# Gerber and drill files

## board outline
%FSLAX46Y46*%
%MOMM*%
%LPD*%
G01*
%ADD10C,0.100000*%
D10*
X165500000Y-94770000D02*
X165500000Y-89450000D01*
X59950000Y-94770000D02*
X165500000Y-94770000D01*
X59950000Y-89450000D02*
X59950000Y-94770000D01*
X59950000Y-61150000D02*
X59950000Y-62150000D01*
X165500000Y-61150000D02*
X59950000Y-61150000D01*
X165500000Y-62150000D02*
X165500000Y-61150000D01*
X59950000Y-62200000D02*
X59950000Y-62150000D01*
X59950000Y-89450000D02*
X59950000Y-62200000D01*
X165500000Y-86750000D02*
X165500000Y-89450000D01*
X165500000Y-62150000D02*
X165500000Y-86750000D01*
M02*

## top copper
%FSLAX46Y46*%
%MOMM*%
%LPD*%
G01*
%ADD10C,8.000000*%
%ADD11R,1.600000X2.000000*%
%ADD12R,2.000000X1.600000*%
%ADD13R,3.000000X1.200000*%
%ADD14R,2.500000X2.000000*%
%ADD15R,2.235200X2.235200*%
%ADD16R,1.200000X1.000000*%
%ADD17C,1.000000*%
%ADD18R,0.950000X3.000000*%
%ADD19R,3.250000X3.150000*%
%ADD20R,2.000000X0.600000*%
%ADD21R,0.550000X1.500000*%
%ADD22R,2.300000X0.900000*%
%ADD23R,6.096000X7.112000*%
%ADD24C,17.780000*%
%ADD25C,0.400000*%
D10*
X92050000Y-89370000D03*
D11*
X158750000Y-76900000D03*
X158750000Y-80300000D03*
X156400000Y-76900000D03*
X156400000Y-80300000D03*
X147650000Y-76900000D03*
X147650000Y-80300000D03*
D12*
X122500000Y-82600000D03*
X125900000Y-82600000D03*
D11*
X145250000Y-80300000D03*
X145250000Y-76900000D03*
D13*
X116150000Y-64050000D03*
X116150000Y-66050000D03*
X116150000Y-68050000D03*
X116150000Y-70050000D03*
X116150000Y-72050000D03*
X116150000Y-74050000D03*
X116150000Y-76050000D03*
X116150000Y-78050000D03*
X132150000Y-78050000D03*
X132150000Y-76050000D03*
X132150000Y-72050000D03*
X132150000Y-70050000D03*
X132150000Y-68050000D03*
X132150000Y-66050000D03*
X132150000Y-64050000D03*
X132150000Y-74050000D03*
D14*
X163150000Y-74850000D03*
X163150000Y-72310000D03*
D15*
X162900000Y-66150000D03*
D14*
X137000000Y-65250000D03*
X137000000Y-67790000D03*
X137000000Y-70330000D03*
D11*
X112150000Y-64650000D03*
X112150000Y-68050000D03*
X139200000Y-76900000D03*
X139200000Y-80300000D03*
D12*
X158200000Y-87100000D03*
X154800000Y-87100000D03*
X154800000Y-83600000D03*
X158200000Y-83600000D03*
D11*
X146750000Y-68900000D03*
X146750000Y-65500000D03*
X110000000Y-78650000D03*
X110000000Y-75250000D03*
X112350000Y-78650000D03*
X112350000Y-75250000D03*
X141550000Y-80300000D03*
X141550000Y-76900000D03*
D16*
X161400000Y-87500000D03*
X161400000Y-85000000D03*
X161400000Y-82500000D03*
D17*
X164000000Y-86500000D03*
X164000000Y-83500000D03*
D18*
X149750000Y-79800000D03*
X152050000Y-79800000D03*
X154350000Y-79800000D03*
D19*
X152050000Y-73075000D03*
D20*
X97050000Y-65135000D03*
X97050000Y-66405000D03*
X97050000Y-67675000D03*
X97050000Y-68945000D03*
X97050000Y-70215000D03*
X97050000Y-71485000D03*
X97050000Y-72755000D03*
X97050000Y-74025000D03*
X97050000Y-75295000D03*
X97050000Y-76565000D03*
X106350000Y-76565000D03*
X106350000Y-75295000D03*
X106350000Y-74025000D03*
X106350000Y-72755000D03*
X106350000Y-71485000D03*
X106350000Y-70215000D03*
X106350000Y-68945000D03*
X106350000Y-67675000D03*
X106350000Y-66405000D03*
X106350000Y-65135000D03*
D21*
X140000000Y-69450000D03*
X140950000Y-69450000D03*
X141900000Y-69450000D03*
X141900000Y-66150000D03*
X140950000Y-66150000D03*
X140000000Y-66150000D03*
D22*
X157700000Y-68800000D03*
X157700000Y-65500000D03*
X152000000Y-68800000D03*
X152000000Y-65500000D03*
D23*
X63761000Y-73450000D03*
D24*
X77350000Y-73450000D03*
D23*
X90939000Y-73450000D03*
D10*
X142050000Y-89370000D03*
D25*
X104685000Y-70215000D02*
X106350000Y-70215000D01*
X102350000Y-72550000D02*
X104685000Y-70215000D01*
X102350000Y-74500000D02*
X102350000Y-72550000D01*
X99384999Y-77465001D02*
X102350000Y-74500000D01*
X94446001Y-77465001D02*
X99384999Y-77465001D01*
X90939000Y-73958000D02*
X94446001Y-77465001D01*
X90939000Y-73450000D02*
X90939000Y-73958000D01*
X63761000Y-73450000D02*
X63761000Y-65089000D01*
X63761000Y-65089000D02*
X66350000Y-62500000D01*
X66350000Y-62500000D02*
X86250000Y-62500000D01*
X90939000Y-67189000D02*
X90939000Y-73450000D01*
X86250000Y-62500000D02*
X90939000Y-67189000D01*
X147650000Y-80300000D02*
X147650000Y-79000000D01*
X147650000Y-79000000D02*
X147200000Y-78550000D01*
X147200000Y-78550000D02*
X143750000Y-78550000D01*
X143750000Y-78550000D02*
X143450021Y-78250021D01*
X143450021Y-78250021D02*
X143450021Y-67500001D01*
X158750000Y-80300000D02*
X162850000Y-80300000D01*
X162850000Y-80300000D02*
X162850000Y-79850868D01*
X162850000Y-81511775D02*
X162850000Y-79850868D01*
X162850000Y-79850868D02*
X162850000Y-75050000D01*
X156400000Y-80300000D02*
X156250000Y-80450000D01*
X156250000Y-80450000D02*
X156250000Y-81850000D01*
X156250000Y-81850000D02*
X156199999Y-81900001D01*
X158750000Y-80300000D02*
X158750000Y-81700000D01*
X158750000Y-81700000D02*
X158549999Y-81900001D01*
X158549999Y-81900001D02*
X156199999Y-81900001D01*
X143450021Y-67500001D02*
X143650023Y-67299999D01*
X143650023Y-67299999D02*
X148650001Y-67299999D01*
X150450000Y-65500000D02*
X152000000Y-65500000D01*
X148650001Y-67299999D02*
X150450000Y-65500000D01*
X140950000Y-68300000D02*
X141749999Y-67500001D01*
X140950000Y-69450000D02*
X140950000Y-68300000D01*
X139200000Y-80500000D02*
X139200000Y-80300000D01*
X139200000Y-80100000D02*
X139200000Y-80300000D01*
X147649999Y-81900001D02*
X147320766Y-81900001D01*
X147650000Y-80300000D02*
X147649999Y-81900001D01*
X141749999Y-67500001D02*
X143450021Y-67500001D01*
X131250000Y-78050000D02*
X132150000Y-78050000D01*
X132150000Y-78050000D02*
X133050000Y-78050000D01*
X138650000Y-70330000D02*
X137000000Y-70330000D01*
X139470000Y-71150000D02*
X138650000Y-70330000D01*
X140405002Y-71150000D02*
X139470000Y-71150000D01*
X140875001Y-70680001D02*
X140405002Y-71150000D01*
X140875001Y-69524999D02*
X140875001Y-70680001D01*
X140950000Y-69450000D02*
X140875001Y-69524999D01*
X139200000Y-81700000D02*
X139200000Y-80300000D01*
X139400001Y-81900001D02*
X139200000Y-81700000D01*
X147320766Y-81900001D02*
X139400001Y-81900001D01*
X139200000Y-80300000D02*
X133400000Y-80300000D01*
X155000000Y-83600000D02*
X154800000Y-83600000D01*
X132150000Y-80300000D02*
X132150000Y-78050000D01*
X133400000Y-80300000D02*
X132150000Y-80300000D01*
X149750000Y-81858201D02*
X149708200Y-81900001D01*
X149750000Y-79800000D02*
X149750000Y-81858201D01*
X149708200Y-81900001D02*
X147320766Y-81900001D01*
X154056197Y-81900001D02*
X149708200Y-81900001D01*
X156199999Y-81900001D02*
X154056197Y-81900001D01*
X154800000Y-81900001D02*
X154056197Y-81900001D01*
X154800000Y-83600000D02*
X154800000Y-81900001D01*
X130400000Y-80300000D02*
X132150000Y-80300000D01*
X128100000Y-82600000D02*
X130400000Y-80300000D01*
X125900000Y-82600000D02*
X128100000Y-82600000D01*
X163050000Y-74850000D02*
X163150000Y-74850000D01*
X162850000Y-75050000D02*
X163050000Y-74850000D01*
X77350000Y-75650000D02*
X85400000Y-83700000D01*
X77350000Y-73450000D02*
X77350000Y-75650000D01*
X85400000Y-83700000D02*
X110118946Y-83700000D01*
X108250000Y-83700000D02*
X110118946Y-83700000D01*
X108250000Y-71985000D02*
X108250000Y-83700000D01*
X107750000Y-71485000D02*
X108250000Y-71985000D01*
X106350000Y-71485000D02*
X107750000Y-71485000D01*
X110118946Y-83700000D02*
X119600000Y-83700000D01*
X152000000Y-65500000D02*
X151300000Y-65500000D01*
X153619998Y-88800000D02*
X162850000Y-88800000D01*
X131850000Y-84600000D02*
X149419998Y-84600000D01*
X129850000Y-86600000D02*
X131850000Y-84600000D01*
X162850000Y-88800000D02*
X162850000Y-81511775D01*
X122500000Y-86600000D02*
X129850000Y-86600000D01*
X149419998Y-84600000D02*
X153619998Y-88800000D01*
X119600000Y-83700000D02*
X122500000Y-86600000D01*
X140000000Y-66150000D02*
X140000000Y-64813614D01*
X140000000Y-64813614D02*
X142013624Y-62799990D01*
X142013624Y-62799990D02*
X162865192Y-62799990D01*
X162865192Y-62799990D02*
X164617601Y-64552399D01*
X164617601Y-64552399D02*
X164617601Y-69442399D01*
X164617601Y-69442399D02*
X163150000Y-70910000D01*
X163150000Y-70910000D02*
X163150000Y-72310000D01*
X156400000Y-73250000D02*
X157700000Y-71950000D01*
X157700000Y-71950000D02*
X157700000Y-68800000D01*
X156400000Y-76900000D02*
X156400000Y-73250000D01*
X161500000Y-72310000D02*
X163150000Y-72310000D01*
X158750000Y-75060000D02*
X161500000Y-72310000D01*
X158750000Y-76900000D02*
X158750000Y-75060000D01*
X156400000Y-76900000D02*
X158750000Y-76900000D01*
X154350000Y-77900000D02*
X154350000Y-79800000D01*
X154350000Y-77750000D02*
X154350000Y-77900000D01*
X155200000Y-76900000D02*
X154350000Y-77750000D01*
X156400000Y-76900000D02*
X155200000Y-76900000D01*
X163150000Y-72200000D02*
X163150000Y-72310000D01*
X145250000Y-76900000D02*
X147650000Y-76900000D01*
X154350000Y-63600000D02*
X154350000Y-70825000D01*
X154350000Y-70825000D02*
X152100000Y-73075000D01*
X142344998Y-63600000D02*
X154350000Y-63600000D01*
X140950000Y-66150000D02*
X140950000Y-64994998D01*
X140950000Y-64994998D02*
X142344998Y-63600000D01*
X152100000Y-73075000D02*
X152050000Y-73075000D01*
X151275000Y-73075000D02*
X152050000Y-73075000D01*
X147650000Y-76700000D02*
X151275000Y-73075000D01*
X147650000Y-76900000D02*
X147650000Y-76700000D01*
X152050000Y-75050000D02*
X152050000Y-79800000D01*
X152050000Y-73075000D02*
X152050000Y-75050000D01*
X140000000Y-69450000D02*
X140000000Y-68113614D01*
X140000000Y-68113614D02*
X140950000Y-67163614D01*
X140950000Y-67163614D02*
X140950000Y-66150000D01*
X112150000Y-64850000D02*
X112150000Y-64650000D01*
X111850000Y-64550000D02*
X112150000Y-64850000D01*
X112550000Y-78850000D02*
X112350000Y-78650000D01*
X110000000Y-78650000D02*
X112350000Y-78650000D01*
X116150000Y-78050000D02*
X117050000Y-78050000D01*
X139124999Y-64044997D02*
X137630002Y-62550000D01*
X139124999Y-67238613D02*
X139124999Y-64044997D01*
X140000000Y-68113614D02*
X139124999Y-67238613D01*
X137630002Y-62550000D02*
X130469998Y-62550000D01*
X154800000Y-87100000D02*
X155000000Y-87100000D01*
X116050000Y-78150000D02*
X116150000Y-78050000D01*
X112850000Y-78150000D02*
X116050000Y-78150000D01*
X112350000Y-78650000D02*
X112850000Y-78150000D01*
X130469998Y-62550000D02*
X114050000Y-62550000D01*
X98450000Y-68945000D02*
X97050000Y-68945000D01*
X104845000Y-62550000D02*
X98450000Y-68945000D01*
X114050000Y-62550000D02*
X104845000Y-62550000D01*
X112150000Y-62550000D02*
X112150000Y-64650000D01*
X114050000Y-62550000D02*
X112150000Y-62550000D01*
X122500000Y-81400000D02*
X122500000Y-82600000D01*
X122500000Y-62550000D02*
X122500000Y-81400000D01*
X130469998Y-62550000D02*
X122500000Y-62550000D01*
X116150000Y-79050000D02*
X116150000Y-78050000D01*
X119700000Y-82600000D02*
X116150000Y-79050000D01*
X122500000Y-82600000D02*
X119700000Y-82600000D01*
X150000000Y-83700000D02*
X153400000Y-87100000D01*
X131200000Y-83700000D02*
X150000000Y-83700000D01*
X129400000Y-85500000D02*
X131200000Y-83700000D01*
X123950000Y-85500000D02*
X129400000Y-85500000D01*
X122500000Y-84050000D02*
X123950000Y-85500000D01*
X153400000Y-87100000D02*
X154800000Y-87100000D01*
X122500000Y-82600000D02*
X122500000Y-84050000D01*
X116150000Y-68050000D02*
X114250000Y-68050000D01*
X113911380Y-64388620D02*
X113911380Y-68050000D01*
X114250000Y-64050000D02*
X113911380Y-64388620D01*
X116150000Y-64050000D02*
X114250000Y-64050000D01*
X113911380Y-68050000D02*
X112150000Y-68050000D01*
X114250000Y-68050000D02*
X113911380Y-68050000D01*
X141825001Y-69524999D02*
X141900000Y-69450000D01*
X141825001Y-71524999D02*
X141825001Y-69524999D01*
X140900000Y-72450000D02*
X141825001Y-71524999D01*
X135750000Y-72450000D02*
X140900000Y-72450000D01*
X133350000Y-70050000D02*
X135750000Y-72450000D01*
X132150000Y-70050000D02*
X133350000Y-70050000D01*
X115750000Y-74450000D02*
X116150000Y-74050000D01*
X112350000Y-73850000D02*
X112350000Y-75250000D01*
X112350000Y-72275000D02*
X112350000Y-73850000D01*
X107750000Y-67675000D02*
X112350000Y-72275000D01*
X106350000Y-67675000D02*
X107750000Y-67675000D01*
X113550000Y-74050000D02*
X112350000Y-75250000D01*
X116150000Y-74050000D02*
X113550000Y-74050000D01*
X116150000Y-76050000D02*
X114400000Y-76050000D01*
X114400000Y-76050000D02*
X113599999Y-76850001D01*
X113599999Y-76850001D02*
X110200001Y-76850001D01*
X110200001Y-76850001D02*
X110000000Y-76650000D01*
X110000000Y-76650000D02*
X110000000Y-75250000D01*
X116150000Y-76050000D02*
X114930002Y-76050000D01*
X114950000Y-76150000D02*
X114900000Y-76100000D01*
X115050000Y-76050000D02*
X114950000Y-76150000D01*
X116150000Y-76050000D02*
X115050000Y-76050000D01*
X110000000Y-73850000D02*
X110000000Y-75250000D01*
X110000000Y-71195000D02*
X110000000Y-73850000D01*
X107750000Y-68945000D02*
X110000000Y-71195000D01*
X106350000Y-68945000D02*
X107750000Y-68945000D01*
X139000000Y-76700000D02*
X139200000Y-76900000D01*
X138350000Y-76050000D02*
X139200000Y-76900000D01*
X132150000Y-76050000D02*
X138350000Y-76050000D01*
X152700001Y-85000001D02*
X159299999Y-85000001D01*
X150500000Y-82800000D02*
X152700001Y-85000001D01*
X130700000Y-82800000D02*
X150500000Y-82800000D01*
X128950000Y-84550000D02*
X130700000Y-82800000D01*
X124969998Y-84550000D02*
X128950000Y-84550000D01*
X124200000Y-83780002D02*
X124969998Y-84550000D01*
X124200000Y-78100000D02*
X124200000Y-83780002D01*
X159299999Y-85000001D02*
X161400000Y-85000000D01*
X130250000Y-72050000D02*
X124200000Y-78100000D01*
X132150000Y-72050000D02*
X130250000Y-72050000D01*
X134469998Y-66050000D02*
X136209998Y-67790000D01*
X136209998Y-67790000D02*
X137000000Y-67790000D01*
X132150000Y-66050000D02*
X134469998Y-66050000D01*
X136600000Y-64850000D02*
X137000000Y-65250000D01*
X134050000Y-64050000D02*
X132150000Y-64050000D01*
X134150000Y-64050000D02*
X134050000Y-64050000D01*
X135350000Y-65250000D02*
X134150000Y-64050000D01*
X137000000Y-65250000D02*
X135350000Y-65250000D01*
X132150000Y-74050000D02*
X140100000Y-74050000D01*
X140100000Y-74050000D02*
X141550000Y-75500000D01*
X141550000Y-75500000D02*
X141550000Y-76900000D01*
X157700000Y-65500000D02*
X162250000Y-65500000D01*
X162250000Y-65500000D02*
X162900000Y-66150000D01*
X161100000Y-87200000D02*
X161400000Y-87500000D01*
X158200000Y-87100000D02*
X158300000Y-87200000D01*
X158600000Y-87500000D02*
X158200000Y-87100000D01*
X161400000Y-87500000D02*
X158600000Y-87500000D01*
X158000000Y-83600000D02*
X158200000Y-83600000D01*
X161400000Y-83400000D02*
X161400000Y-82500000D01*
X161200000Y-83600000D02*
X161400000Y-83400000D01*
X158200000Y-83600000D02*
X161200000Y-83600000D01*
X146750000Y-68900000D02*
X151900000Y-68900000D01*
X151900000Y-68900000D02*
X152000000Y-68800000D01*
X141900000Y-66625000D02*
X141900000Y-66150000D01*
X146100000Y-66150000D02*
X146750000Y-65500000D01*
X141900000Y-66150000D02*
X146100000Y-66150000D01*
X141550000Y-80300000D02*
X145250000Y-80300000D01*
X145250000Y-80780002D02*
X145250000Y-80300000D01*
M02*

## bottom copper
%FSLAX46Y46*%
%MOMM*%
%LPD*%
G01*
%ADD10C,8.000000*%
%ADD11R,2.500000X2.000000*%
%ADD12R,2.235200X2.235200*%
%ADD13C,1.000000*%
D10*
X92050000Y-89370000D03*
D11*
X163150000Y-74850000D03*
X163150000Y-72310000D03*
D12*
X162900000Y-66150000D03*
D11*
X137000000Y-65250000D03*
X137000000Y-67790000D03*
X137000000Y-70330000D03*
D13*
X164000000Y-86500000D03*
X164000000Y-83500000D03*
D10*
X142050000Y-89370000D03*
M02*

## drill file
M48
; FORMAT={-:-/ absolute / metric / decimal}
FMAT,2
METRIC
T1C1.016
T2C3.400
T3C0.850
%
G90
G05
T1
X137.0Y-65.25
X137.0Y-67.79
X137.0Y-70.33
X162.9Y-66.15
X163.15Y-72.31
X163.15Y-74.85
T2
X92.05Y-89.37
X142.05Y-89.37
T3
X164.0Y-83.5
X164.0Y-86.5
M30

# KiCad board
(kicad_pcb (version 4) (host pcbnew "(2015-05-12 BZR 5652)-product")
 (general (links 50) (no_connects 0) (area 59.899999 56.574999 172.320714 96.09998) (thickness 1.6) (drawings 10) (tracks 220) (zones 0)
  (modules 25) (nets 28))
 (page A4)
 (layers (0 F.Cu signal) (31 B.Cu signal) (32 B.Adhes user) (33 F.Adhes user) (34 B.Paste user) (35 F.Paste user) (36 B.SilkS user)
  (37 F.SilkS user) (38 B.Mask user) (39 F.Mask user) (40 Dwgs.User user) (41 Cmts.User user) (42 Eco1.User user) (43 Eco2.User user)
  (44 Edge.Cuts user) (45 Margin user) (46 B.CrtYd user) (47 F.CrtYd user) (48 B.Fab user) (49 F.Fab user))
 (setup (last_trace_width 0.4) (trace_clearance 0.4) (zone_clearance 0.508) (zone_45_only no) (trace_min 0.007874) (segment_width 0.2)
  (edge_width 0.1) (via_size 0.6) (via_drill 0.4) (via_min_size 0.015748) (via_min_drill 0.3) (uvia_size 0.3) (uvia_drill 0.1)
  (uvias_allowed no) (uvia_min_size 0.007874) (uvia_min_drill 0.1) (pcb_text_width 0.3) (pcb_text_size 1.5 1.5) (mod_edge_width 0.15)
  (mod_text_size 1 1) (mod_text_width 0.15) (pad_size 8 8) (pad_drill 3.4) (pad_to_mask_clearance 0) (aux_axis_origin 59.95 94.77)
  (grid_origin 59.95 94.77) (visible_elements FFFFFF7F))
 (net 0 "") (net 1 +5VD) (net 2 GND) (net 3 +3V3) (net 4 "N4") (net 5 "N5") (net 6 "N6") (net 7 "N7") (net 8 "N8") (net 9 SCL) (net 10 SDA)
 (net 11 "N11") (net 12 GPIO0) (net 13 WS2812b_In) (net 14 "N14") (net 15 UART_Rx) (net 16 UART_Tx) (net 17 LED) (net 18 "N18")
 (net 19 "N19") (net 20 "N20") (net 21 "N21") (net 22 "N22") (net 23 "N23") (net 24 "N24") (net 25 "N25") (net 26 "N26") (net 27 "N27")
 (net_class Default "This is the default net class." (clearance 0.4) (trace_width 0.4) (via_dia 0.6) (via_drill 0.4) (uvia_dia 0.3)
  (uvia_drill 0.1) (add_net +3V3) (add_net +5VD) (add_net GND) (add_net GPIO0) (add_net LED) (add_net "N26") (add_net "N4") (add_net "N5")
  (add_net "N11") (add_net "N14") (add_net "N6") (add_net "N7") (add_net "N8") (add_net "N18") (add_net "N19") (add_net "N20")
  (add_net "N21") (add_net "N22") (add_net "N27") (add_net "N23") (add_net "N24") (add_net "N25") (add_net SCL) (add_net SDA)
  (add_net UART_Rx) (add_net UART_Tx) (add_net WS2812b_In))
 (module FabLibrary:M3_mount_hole (layer F.Cu) (at 92.05 89.37)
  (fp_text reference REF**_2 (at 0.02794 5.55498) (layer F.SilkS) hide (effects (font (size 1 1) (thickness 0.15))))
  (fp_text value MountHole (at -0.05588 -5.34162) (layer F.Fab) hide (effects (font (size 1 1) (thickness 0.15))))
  (pad 1 thru_hole circle (at 0 0) (size 8 8) (drill 3.4) (layers *.Cu *.Mask F.SilkS)))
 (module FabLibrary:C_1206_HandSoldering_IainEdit (layer F.Cu) (at 158.75 78.6 270)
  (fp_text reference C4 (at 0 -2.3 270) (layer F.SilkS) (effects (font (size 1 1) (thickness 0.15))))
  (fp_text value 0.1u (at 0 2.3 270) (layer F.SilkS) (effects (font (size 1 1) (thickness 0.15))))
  (pad 1 smd rect (at -1.7 0 270) (size 2 1.6) (layers F.Cu F.Paste F.Mask) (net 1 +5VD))
  (pad 2 smd rect (at 1.7 0 270) (size 2 1.6) (layers F.Cu F.Paste F.Mask) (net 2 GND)))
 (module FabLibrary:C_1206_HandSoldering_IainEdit (layer F.Cu) (at 156.4 78.6 270)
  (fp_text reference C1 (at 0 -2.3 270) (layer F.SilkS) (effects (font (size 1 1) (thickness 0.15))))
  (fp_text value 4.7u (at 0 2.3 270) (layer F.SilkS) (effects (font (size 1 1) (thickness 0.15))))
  (pad 1 smd rect (at -1.7 0 270) (size 2 1.6) (layers F.Cu F.Paste F.Mask) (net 1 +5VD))
  (pad 2 smd rect (at 1.7 0 270) (size 2 1.6) (layers F.Cu F.Paste F.Mask) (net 2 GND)))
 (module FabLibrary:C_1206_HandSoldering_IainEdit (layer F.Cu) (at 147.65 78.6 270)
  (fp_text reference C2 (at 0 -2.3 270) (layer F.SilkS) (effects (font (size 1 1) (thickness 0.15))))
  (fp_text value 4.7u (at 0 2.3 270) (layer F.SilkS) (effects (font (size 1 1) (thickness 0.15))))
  (pad 1 smd rect (at -1.7 0 270) (size 2 1.6) (layers F.Cu F.Paste F.Mask) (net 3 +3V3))
  (pad 2 smd rect (at 1.7 0 270) (size 2 1.6) (layers F.Cu F.Paste F.Mask) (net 2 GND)))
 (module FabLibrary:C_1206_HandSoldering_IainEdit (layer F.Cu) (at 124.2 82.6)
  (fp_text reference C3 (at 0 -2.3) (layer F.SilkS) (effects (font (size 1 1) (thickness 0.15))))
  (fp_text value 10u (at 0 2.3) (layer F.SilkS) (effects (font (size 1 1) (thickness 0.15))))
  (pad 1 smd rect (at -1.7 0) (size 2 1.6) (layers F.Cu F.Paste F.Mask) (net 3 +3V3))
  (pad 2 smd rect (at 1.7 0) (size 2 1.6) (layers F.Cu F.Paste F.Mask) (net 2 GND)))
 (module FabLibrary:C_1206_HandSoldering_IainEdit (layer F.Cu) (at 145.25 78.6 90)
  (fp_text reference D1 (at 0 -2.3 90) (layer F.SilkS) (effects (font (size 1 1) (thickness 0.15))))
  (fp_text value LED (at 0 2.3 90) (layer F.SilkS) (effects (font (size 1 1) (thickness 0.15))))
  (pad 1 smd rect (at -1.7 0 90) (size 2 1.6) (layers F.Cu F.Paste F.Mask) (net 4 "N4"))
  (pad 2 smd rect (at 1.7 0 90) (size 2 1.6) (layers F.Cu F.Paste F.Mask) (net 3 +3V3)))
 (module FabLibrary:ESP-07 (layer F.Cu) (at 124.15 70.05 270)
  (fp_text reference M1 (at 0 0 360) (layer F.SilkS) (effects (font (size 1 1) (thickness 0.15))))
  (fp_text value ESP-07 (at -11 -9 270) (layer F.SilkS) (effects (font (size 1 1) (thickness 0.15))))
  (pad 1 smd rect (at -6 8 270) (size 1.2 3) (layers F.Cu F.Paste F.Mask) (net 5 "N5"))
  (pad 2 smd rect (at -4 8 270) (size 1.2 3) (layers F.Cu F.Paste F.Mask) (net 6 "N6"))
  (pad 3 smd rect (at -2 8 270) (size 1.2 3) (layers F.Cu F.Paste F.Mask) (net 5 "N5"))
  (pad 4 smd rect (at 0 8 270) (size 1.2 3) (layers F.Cu F.Paste F.Mask) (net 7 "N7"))
  (pad 5 smd rect (at 2 8 270) (size 1.2 3) (layers F.Cu F.Paste F.Mask) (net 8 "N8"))
  (pad 6 smd rect (at 4 8 270) (size 1.2 3) (layers F.Cu F.Paste F.Mask) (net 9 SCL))
  (pad 7 smd rect (at 6 8 270) (size 1.2 3) (layers F.Cu F.Paste F.Mask) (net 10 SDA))
  (pad 8 smd rect (at 8 8 270) (size 1.2 3) (layers F.Cu F.Paste F.Mask) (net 3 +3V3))
  (pad 9 smd rect (at 8 -8 270) (size 1.2 3) (layers F.Cu F.Paste F.Mask) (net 2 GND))
  (pad 10 smd rect (at 6 -8 270) (size 1.2 3) (layers F.Cu F.Paste F.Mask) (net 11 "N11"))
  (pad 12 smd rect (at 2 -8 270) (size 1.2 3) (layers F.Cu F.Paste F.Mask) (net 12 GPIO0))
  (pad 13 smd rect (at 0 -8 270) (size 1.2 3) (layers F.Cu F.Paste F.Mask) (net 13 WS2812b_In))
  (pad 14 smd rect (at -2 -8 270) (size 1.2 3) (layers F.Cu F.Paste F.Mask) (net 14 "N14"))
  (pad 15 smd rect (at -4 -8 270) (size 1.2 3) (layers F.Cu F.Paste F.Mask) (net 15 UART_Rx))
  (pad 16 smd rect (at -6 -8 270) (size 1.2 3) (layers F.Cu F.Paste F.Mask) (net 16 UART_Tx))
  (pad 11 smd rect (at 4 -8 270) (size 1.2 3) (layers F.Cu F.Paste F.Mask) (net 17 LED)))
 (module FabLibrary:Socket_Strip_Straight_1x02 (layer F.Cu) (at 163.15 74.85 90)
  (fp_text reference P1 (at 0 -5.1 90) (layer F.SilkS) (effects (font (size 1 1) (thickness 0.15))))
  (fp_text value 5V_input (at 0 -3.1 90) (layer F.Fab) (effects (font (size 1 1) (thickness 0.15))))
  (pad 1 thru_hole rect (at 0 0 90) (size 2 2.5) (drill 1.016) (layers *.Mask F.Cu F.SilkS) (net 2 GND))
  (pad 2 thru_hole rect (at 2.54 0 90) (size 2 2.5) (drill 1.016) (layers *.Mask F.Cu F.SilkS) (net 1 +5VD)))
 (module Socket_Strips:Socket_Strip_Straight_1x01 (layer F.Cu) (at 162.9 66.15)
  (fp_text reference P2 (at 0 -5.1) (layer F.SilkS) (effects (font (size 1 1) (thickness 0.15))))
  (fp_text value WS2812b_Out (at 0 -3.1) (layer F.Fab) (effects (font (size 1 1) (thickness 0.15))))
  (pad 1 thru_hole rect (at 0 0) (size 2.2352 2.2352) (drill 1.016) (layers *.Cu *.Mask F.SilkS) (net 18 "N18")))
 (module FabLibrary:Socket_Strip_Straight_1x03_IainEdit (layer F.Cu) (at 137 65.25 270)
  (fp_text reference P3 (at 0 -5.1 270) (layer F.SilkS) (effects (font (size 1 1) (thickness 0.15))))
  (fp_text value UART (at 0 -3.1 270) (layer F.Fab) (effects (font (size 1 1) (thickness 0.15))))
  (pad 1 thru_hole rect (at 0 0 270) (size 2 2.5) (drill 1.016) (layers *.Mask F.Cu F.SilkS) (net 16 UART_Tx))
  (pad 2 thru_hole rect (at 2.54 0 270) (size 2 2.5) (drill 1.016) (layers *.Mask F.Cu F.SilkS) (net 15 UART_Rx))
  (pad 3 thru_hole rect (at 5.08 0 270) (size 2 2.5) (drill 1.016) (layers *.Mask F.Cu F.SilkS) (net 2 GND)))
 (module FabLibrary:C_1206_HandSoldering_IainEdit (layer F.Cu) (at 112.15 66.35 270)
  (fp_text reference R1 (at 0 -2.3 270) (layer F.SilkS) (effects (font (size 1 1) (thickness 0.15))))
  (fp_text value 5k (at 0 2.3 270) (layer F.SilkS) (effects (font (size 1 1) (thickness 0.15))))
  (pad 1 smd rect (at -1.7 0 270) (size 2 1.6) (layers F.Cu F.Paste F.Mask) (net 3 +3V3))
  (pad 2 smd rect (at 1.7 0 270) (size 2 1.6) (layers F.Cu F.Paste F.Mask) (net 5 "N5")))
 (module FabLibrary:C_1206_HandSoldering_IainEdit (layer F.Cu) (at 139.2 78.6 270)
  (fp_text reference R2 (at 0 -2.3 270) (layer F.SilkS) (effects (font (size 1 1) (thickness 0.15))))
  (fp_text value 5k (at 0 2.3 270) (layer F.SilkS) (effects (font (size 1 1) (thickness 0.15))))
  (pad 1 smd rect (at -1.7 0 270) (size 2 1.6) (layers F.Cu F.Paste F.Mask) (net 11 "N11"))
  (pad 2 smd rect (at 1.7 0 270) (size 2 1.6) (layers F.Cu F.Paste F.Mask) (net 2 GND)))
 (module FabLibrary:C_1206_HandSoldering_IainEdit (layer F.Cu) (at 156.5 87.1 180)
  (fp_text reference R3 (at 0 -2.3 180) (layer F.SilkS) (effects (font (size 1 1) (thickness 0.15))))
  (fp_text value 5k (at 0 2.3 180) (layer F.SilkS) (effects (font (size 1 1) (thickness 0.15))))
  (pad 1 smd rect (at -1.7 0 180) (size 2 1.6) (layers F.Cu F.Paste F.Mask) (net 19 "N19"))
  (pad 2 smd rect (at 1.7 0 180) (size 2 1.6) (layers F.Cu F.Paste F.Mask) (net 3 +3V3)))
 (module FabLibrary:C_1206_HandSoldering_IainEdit (layer F.Cu) (at 156.5 83.6)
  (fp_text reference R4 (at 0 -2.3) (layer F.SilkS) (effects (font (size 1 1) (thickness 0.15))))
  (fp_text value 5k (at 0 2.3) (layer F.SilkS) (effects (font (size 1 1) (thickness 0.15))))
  (pad 1 smd rect (at -1.7 0) (size 2 1.6) (layers F.Cu F.Paste F.Mask) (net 2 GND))
  (pad 2 smd rect (at 1.7 0) (size 2 1.6) (layers F.Cu F.Paste F.Mask) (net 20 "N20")))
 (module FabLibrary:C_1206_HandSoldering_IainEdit (layer F.Cu) (at 146.75 67.2 90)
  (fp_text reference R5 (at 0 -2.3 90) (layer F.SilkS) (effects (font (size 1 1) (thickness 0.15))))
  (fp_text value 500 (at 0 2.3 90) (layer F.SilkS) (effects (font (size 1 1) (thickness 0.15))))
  (pad 1 smd rect (at -1.7 0 90) (size 2 1.6) (layers F.Cu F.Paste F.Mask) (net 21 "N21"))
  (pad 2 smd rect (at 1.7 0 90) (size 2 1.6) (layers F.Cu F.Paste F.Mask) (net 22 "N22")))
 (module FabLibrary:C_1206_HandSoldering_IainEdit (layer F.Cu) (at 110 76.95 90)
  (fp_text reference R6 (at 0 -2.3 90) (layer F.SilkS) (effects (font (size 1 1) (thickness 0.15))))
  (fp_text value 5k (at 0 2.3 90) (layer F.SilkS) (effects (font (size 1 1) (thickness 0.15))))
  (pad 1 smd rect (at -1.7 0 90) (size 2 1.6) (layers F.Cu F.Paste F.Mask) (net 3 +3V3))
  (pad 2 smd rect (at 1.7 0 90) (size 2 1.6) (layers F.Cu F.Paste F.Mask) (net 10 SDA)))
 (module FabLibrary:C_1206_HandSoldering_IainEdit (layer F.Cu) (at 112.35 76.95 90)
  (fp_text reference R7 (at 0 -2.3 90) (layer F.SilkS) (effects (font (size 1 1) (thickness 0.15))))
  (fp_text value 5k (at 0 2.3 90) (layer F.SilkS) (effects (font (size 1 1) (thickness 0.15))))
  (pad 1 smd rect (at -1.7 0 90) (size 2 1.6) (layers F.Cu F.Paste F.Mask) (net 3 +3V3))
  (pad 2 smd rect (at 1.7 0 90) (size 2 1.6) (layers F.Cu F.Paste F.Mask) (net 9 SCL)))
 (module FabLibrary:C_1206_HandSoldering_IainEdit (layer F.Cu) (at 141.55 78.6 90)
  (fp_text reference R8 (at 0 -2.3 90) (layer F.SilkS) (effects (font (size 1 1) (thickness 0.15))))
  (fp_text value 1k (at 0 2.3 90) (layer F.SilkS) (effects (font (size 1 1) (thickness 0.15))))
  (pad 1 smd rect (at -1.7 0 90) (size 2 1.6) (layers F.Cu F.Paste F.Mask) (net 4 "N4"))
  (pad 2 smd rect (at 1.7 0 90) (size 2 1.6) (layers F.Cu F.Paste F.Mask) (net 17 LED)))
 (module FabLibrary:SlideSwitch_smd (layer F.Cu) (at 164 85 90)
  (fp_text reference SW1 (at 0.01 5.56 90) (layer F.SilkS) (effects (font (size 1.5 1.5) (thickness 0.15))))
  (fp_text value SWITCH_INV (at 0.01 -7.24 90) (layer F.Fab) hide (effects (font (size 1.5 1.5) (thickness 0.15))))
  (pad 1 smd rect (at -2.5 -2.6 90) (size 1 1.2) (layers F.Cu F.Paste F.Mask) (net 19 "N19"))
  (pad 2 smd rect (at 0 -2.6 90) (size 1 1.2) (layers F.Cu F.Paste F.Mask) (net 12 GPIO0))
  (pad 3 smd rect (at 2.5 -2.6 90) (size 1 1.2) (layers F.Cu F.Paste F.Mask) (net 20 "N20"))
  (pad "" np_thru_hole circle (at -1.5 0 90) (size 1 1) (drill 0.85) (layers *.Cu *.Mask F.SilkS))
  (pad "" np_thru_hole circle (at 1.5 0 90) (size 1 1) (drill 0.85) (layers *.Cu *.Mask F.SilkS)))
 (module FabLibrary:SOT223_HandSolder (layer F.Cu) (at 152.05 78.3)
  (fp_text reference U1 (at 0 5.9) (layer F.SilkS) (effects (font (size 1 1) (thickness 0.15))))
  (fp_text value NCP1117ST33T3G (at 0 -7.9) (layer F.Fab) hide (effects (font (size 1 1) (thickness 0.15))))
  (pad 1 smd rect (at -2.3 1.5) (size 0.95 3) (layers F.Cu F.Paste F.Mask) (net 2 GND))
  (pad 2 smd rect (at 0 1.5) (size 0.95 3) (layers F.Cu F.Paste F.Mask) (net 3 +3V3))
  (pad 3 smd rect (at 2.3 1.5) (size 0.95 3) (layers F.Cu F.Paste F.Mask) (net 1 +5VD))
  (pad 2 smd rect (at 0 -5.225) (size 3.25 3.15) (layers F.Cu F.Paste F.Mask) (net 3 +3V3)))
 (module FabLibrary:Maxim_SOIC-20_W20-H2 (layer F.Cu) (at 101.7 70.85 270)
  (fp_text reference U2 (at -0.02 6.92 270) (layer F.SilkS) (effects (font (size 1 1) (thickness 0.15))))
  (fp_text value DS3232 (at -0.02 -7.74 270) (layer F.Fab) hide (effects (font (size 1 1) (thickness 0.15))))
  (pad 1 smd rect (at -5.715 4.65 270) (size 0.6 2) (layers F.Cu F.Paste F.Mask))
  (pad 2 smd rect (at -4.445 4.65 270) (size 0.6 2) (layers F.Cu F.Paste F.Mask))
  (pad 3 smd rect (at -3.175 4.65 270) (size 0.6 2) (layers F.Cu F.Paste F.Mask) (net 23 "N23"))
  (pad 4 smd rect (at -1.905 4.65 270) (size 0.6 2) (layers F.Cu F.Paste F.Mask) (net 3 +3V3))
  (pad 5 smd rect (at -0.635 4.65 270) (size 0.6 2) (layers F.Cu F.Paste F.Mask) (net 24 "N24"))
  (pad 6 smd rect (at 0.635 4.65 270) (size 0.6 2) (layers F.Cu F.Paste F.Mask) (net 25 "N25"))
  (pad 7 smd rect (at 1.905 4.65 270) (size 0.6 2) (layers F.Cu F.Paste F.Mask))
  (pad 8 smd rect (at 3.175 4.65 270) (size 0.6 2) (layers F.Cu F.Paste F.Mask))
  (pad 9 smd rect (at 4.445 4.65 270) (size 0.6 2) (layers F.Cu F.Paste F.Mask))
  (pad 10 smd rect (at 5.715 4.65 270) (size 0.6 2) (layers F.Cu F.Paste F.Mask))
  (pad 11 smd rect (at 5.715 -4.65 270) (size 0.6 2) (layers F.Cu F.Paste F.Mask))
  (pad 12 smd rect (at 4.445 -4.65 270) (size 0.6 2) (layers F.Cu F.Paste F.Mask))
  (pad 13 smd rect (at 3.175 -4.65 270) (size 0.6 2) (layers F.Cu F.Paste F.Mask))
  (pad 14 smd rect (at 1.905 -4.65 270) (size 0.6 2) (layers F.Cu F.Paste F.Mask))
  (pad 15 smd rect (at 0.635 -4.65 270) (size 0.6 2) (layers F.Cu F.Paste F.Mask) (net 2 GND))
  (pad 16 smd rect (at -0.635 -4.65 270) (size 0.6 2) (layers F.Cu F.Paste F.Mask) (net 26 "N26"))
  (pad 17 smd rect (at -1.905 -4.65 270) (size 0.6 2) (layers F.Cu F.Paste F.Mask) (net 10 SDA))
  (pad 18 smd rect (at -3.175 -4.65 270) (size 0.6 2) (layers F.Cu F.Paste F.Mask) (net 9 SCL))
  (pad 19 smd rect (at -4.445 -4.65 270) (size 0.6 2) (layers F.Cu F.Paste F.Mask))
  (pad 20 smd rect (at -5.715 -4.65 270) (size 0.6 2) (layers F.Cu F.Paste F.Mask) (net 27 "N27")))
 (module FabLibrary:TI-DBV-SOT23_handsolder (layer F.Cu) (at 140.95 67.85)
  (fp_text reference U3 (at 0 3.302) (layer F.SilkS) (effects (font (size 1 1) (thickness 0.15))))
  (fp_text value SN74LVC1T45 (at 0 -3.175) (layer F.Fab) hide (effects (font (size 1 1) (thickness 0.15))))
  (pad 1 smd rect (at -0.95 1.6) (size 0.55 1.5) (layers F.Cu F.Paste F.Mask) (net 3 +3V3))
  (pad 2 smd rect (at 0 1.6) (size 0.55 1.5) (layers F.Cu F.Paste F.Mask) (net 2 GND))
  (pad 3 smd rect (at 0.95 1.6) (size 0.55 1.5) (layers F.Cu F.Paste F.Mask) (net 13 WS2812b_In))
  (pad 4 smd rect (at 0.95 -1.7) (size 0.55 1.5) (layers F.Cu F.Paste F.Mask) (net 22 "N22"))
  (pad 5 smd rect (at 0 -1.7) (size 0.55 1.5) (layers F.Cu F.Paste F.Mask) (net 3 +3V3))
  (pad 6 smd rect (at -0.95 -1.7) (size 0.55 1.5) (layers F.Cu F.Paste F.Mask) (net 1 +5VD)))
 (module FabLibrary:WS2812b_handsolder (layer F.Cu) (at 154.85 67.15 180)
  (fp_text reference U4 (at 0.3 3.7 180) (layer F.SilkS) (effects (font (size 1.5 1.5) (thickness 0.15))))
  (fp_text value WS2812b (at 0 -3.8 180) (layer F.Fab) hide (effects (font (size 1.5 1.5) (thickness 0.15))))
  (pad 1 smd rect (at -2.85 -1.65 180) (size 2.3 0.9) (layers F.Cu F.Paste F.Mask) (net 1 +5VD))
  (pad 2 smd rect (at -2.85 1.65 180) (size 2.3 0.9) (layers F.Cu F.Paste F.Mask) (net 18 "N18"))
  (pad 4 smd rect (at 2.85 -1.65 180) (size 2.3 0.9) (layers F.Cu F.Paste F.Mask) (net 21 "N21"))
  (pad 3 smd rect (at 2.85 1.65 180) (size 2.3 0.9) (layers F.Cu F.Paste F.Mask) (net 2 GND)))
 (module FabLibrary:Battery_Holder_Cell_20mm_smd (layer F.Cu) (at 77.35 73.45 180)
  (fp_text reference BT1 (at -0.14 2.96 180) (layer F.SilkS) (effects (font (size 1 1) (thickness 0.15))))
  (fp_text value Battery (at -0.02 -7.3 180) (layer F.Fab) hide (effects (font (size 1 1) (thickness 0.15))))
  (pad 1 smd rect (at 13.589 0 180) (size 6.096 7.112) (layers F.Cu F.Paste F.Mask) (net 26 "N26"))
  (pad 2 smd circle (at 0 0 180) (size 17.78 17.78) (layers F.Cu F.Paste F.Mask) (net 2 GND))
  (pad 1 smd rect (at -13.589 0 180) (size 6.096 7.112) (layers F.Cu F.Paste F.Mask) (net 26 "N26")))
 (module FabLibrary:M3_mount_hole (layer F.Cu) (at 142.05 89.37)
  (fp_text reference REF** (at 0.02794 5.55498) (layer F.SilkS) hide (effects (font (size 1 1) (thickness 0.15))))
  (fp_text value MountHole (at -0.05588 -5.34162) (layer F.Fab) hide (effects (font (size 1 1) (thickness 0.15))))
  (pad 1 thru_hole circle (at 0 0) (size 8 8) (drill 3.4) (layers *.Cu *.Mask F.SilkS)))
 (gr_line (start 165.5 94.77) (end 165.5 89.45) (angle 90) (layer Edge.Cuts) (width 0.1))
 (gr_line (start 59.95 94.77) (end 165.5 94.77) (angle 90) (layer Edge.Cuts) (width 0.1))
 (gr_line (start 59.95 89.45) (end 59.95 94.77) (angle 90) (layer Edge.Cuts) (width 0.1))
 (gr_line (start 59.95 61.15) (end 59.95 62.15) (angle 90) (layer Edge.Cuts) (width 0.1))
 (gr_line (start 165.5 61.15) (end 59.95 61.15) (angle 90) (layer Edge.Cuts) (width 0.1))
 (gr_line (start 165.5 62.15) (end 165.5 61.15) (angle 90) (layer Edge.Cuts) (width 0.1))
 (gr_line (start 59.95 62.2) (end 59.95 62.15) (layer Edge.Cuts) (width 0.1))
 (gr_line (start 59.95 89.45) (end 59.95 62.2) (layer Edge.Cuts) (width 0.1))
 (gr_line (start 165.5 86.75) (end 165.5 89.45) (layer Edge.Cuts) (width 0.1))
 (gr_line (start 165.5 62.15) (end 165.5 86.75) (layer Edge.Cuts) (width 0.1))
 (segment (start 104.685 70.215) (end 106.35 70.215) (width 0.4) (layer F.Cu) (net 26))
 (segment (start 102.35 72.55) (end 104.685 70.215) (width 0.4) (layer F.Cu) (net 26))
 (segment (start 102.35 74.5) (end 102.35 72.55) (width 0.4) (layer F.Cu) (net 26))
 (segment (start 99.384999 77.465001) (end 102.35 74.5) (width 0.4) (layer F.Cu) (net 26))
 (segment (start 94.446001 77.465001) (end 99.384999 77.465001) (width 0.4) (layer F.Cu) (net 26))
 (segment (start 90.939 73.958) (end 94.446001 77.465001) (width 0.4) (layer F.Cu) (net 26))
 (segment (start 90.939 73.45) (end 90.939 73.958) (width 0.4) (layer F.Cu) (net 26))
 (segment (start 63.761 73.45) (end 63.761 65.089) (width 0.4) (layer F.Cu) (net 26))
 (segment (start 63.761 65.089) (end 66.35 62.5) (width 0.4) (layer F.Cu) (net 26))
 (segment (start 66.35 62.5) (end 86.25 62.5) (width 0.4) (layer F.Cu) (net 26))
 (segment (start 90.939 67.189) (end 90.939 73.45) (width 0.4) (layer F.Cu) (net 26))
 (segment (start 86.25 62.5) (end 90.939 67.189) (width 0.4) (layer F.Cu) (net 26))
 (segment (start 147.65 80.3) (end 147.65 79) (width 0.4) (layer F.Cu) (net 2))
 (segment (start 147.65 79) (end 147.2 78.55) (width 0.4) (layer F.Cu) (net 2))
 (segment (start 147.2 78.55) (end 143.75 78.55) (width 0.4) (layer F.Cu) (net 2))
 (segment (start 143.75 78.55) (end 143.450021 78.250021) (width 0.4) (layer F.Cu) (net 2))
 (segment (start 143.450021 78.250021) (end 143.450021 67.500001) (width 0.4) (layer F.Cu) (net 2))
 (segment (start 158.75 80.3) (end 162.85 80.3) (width 0.4) (layer F.Cu) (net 2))
 (segment (start 162.85 80.3) (end 162.85 79.850868) (width 0.4) (layer F.Cu) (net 2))
 (segment (start 162.85 81.511775) (end 162.85 79.850868) (width 0.4) (layer F.Cu) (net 2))
 (segment (start 162.85 79.850868) (end 162.85 75.05) (width 0.4) (layer F.Cu) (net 2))
 (segment (start 156.4 80.3) (end 156.25 80.45) (width 0.4) (layer F.Cu) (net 2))
 (segment (start 156.25 80.45) (end 156.25 81.85) (width 0.4) (layer F.Cu) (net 2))
 (segment (start 156.25 81.85) (end 156.199999 81.900001) (width 0.4) (layer F.Cu) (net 2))
 (segment (start 158.75 80.3) (end 158.75 81.7) (width 0.4) (layer F.Cu) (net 2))
 (segment (start 158.75 81.7) (end 158.549999 81.900001) (width 0.4) (layer F.Cu) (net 2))
 (segment (start 158.549999 81.900001) (end 156.199999 81.900001) (width 0.4) (layer F.Cu) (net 2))
 (segment (start 143.450021 67.500001) (end 143.650023 67.299999) (width 0.4) (layer F.Cu) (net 2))
 (segment (start 143.650023 67.299999) (end 148.650001 67.299999) (width 0.4) (layer F.Cu) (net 2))
 (segment (start 150.45 65.5) (end 152 65.5) (width 0.4) (layer F.Cu) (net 2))
 (segment (start 148.650001 67.299999) (end 150.45 65.5) (width 0.4) (layer F.Cu) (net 2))
 (segment (start 140.95 68.3) (end 141.749999 67.500001) (width 0.4) (layer F.Cu) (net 2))
 (segment (start 140.95 69.45) (end 140.95 68.3) (width 0.4) (layer F.Cu) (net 2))
 (segment (start 139.2 80.5) (end 139.2 80.3) (width 0.4) (layer F.Cu) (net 2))
 (segment (start 139.2 80.1) (end 139.2 80.3) (width 0.4) (layer F.Cu) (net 2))
 (segment (start 147.649999 81.900001) (end 147.320766 81.900001) (width 0.4) (layer F.Cu) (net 2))
 (segment (start 147.65 80.3) (end 147.649999 81.900001) (width 0.4) (layer F.Cu) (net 2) (status 10))
 (segment (start 141.749999 67.500001) (end 143.450021 67.500001) (width 0.4) (layer F.Cu) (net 2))
 (segment (start 131.25 78.05) (end 132.15 78.05) (width 0.4) (layer F.Cu) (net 2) (status 30))
 (segment (start 132.15 78.05) (end 133.05 78.05) (width 0.4) (layer F.Cu) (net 2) (status 30))
 (segment (start 138.65 70.33) (end 137 70.33) (width 0.4) (layer F.Cu) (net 2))
 (segment (start 139.47 71.15) (end 138.65 70.33) (width 0.4) (layer F.Cu) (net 2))
 (segment (start 140.405002 71.15) (end 139.47 71.15) (width 0.4) (layer F.Cu) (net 2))
 (segment (start 140.875001 70.680001) (end 140.405002 71.15) (width 0.4) (layer F.Cu) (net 2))
 (segment (start 140.875001 69.524999) (end 140.875001 70.680001) (width 0.4) (layer F.Cu) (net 2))
 (segment (start 140.95 69.45) (end 140.875001 69.524999) (width 0.4) (layer F.Cu) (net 2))
 (segment (start 139.2 81.7) (end 139.2 80.3) (width 0.4) (layer F.Cu) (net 2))
 (segment (start 139.400001 81.900001) (end 139.2 81.7) (width 0.4) (layer F.Cu) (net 2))
 (segment (start 147.320766 81.900001) (end 139.400001 81.900001) (width 0.4) (layer F.Cu) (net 2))
 (segment (start 139.2 80.3) (end 133.4 80.3) (width 0.4) (layer F.Cu) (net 2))
 (segment (start 155 83.6) (end 154.8 83.6) (width 0.4) (layer F.Cu) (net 2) (status 30))
 (segment (start 132.15 80.3) (end 132.15 78.05) (width 0.4) (layer F.Cu) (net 2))
 (segment (start 133.4 80.3) (end 132.15 80.3) (width 0.4) (layer F.Cu) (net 2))
 (segment (start 149.75 81.858201) (end 149.7082 81.900001) (width 0.4) (layer F.Cu) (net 2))
 (segment (start 149.75 79.8) (end 149.75 81.858201) (width 0.4) (layer F.Cu) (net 2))
 (segment (start 149.7082 81.900001) (end 147.320766 81.900001) (width 0.4) (layer F.Cu) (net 2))
 (segment (start 154.056197 81.900001) (end 149.7082 81.900001) (width 0.4) (layer F.Cu) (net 2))
 (segment (start 156.199999 81.900001) (end 154.056197 81.900001) (width 0.4) (layer F.Cu) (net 2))
 (segment (start 154.8 81.900001) (end 154.056197 81.900001) (width 0.4) (layer F.Cu) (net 2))
 (segment (start 154.8 83.6) (end 154.8 81.900001) (width 0.4) (layer F.Cu) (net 2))
 (segment (start 130.4 80.3) (end 132.15 80.3) (width 0.4) (layer F.Cu) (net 2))
 (segment (start 128.1 82.6) (end 130.4 80.3) (width 0.4) (layer F.Cu) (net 2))
 (segment (start 125.9 82.6) (end 128.1 82.6) (width 0.4) (layer F.Cu) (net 2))
 (segment (start 163.05 74.85) (end 163.15 74.85) (width 0.4) (layer F.Cu) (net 2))
 (segment (start 162.85 75.05) (end 163.05 74.85) (width 0.4) (layer F.Cu) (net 2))
 (segment (start 77.35 75.65) (end 85.4 83.7) (width 0.4) (layer F.Cu) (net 2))
 (segment (start 77.35 73.45) (end 77.35 75.65) (width 0.4) (layer F.Cu) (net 2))
 (segment (start 85.4 83.7) (end 110.118946 83.7) (width 0.4) (layer F.Cu) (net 2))
 (segment (start 108.25 83.7) (end 110.118946 83.7) (width 0.4) (layer F.Cu) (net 2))
 (segment (start 108.25 71.985) (end 108.25 83.7) (width 0.4) (layer F.Cu) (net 2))
 (segment (start 107.75 71.485) (end 108.25 71.985) (width 0.4) (layer F.Cu) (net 2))
 (segment (start 106.35 71.485) (end 107.75 71.485) (width 0.4) (layer F.Cu) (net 2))
 (segment (start 110.118946 83.7) (end 119.6 83.7) (width 0.4) (layer F.Cu) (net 2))
 (segment (start 152 65.5) (end 151.3 65.5) (width 0.4) (layer F.Cu) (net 2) (status 30))
 (segment (start 153.619998 88.8) (end 162.85 88.8) (width 0.4) (layer F.Cu) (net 2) (status 20))
 (segment (start 131.85 84.6) (end 149.419998 84.6) (width 0.4) (layer F.Cu) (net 2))
 (segment (start 129.85 86.6) (end 131.85 84.6) (width 0.4) (layer F.Cu) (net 2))
 (segment (start 162.85 88.8) (end 162.85 81.511775) (width 0.4) (layer F.Cu) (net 2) (status 10))
 (segment (start 122.5 86.6) (end 129.85 86.6) (width 0.4) (layer F.Cu) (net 2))
 (segment (start 149.419998 84.6) (end 153.619998 88.8) (width 0.4) (layer F.Cu) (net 2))
 (segment (start 119.6 83.7) (end 122.5 86.6) (width 0.4) (layer F.Cu) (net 2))
 (segment (start 140 66.15) (end 140 64.813614) (width 0.4) (layer F.Cu) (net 1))
 (segment (start 140 64.813614) (end 142.013624 62.79999) (width 0.4) (layer F.Cu) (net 1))
 (segment (start 142.013624 62.79999) (end 162.865192 62.79999) (width 0.4) (layer F.Cu) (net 1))
 (segment (start 162.865192 62.79999) (end 164.617601 64.552399) (width 0.4) (layer F.Cu) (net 1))
 (segment (start 164.617601 64.552399) (end 164.617601 69.442399) (width 0.4) (layer F.Cu) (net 1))
 (segment (start 164.617601 69.442399) (end 163.15 70.91) (width 0.4) (layer F.Cu) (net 1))
 (segment (start 163.15 70.91) (end 163.15 72.31) (width 0.4) (layer F.Cu) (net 1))
 (segment (start 156.4 73.25) (end 157.7 71.95) (width 0.4) (layer F.Cu) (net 1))
 (segment (start 157.7 71.95) (end 157.7 68.8) (width 0.4) (layer F.Cu) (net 1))
 (segment (start 156.4 76.9) (end 156.4 73.25) (width 0.4) (layer F.Cu) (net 1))
 (segment (start 161.5 72.31) (end 163.15 72.31) (width 0.4) (layer F.Cu) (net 1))
 (segment (start 158.75 75.06) (end 161.5 72.31) (width 0.4) (layer F.Cu) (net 1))
 (segment (start 158.75 76.9) (end 158.75 75.06) (width 0.4) (layer F.Cu) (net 1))
 (segment (start 156.4 76.9) (end 158.75 76.9) (width 0.4) (layer F.Cu) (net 1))
 (segment (start 154.35 77.9) (end 154.35 79.8) (width 0.4) (layer F.Cu) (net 1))
 (segment (start 154.35 77.75) (end 154.35 77.9) (width 0.4) (layer F.Cu) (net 1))
 (segment (start 155.2 76.9) (end 154.35 77.75) (width 0.4) (layer F.Cu) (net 1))
 (segment (start 156.4 76.9) (end 155.2 76.9) (width 0.4) (layer F.Cu) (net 1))
 (segment (start 163.15 72.2) (end 163.15 72.31) (width 0.4) (layer F.Cu) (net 1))
 (segment (start 145.25 76.9) (end 147.65 76.9) (width 0.4) (layer F.Cu) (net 3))
 (segment (start 154.35 63.6) (end 154.35 70.825) (width 0.4) (layer F.Cu) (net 3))
 (segment (start 154.35 70.825) (end 152.1 73.075) (width 0.4) (layer F.Cu) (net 3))
 (segment (start 142.344998 63.6) (end 154.35 63.6) (width 0.4) (layer F.Cu) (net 3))
 (segment (start 140.95 66.15) (end 140.95 64.994998) (width 0.4) (layer F.Cu) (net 3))
 (segment (start 140.95 64.994998) (end 142.344998 63.6) (width 0.4) (layer F.Cu) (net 3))
 (segment (start 152.1 73.075) (end 152.05 73.075) (width 0.4) (layer F.Cu) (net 3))
 (segment (start 151.275 73.075) (end 152.05 73.075) (width 0.4) (layer F.Cu) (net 3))
 (segment (start 147.65 76.7) (end 151.275 73.075) (width 0.4) (layer F.Cu) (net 3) (status 10))
 (segment (start 147.65 76.9) (end 147.65 76.7) (width 0.4) (layer F.Cu) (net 3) (status 30))
 (segment (start 152.05 75.05) (end 152.05 79.8) (width 0.4) (layer F.Cu) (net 3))
 (segment (start 152.05 73.075) (end 152.05 75.05) (width 0.4) (layer F.Cu) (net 3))
 (segment (start 140 69.45) (end 140 68.113614) (width 0.4) (layer F.Cu) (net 3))
 (segment (start 140 68.113614) (end 140.95 67.163614) (width 0.4) (layer F.Cu) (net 3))
 (segment (start 140.95 67.163614) (end 140.95 66.15) (width 0.4) (layer F.Cu) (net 3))
 (segment (start 112.15 64.85) (end 112.15 64.65) (width 0.4) (layer F.Cu) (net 3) (status 30))
 (segment (start 111.85 64.55) (end 112.15 64.85) (width 0.4) (layer F.Cu) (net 3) (status 30))
 (segment (start 112.55 78.85) (end 112.35 78.65) (width 0.4) (layer F.Cu) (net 3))
 (segment (start 110 78.65) (end 112.35 78.65) (width 0.4) (layer F.Cu) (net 3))
 (segment (start 116.15 78.05) (end 117.05 78.05) (width 0.4) (layer F.Cu) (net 3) (status 30))
 (segment (start 139.124999 64.044997) (end 137.630002 62.55) (width 0.4) (layer F.Cu) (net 3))
 (segment (start 139.124999 67.238613) (end 139.124999 64.044997) (width 0.4) (layer F.Cu) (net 3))
 (segment (start 140 68.113614) (end 139.124999 67.238613) (width 0.4) (layer F.Cu) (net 3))
 (segment (start 137.630002 62.55) (end 130.469998 62.55) (width 0.4) (layer F.Cu) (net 3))
 (segment (start 154.8 87.1) (end 155 87.1) (width 0.4) (layer F.Cu) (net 3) (status 30))
 (segment (start 116.05 78.15) (end 116.15 78.05) (width 0.4) (layer F.Cu) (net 3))
 (segment (start 112.85 78.15) (end 116.05 78.15) (width 0.4) (layer F.Cu) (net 3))
 (segment (start 112.35 78.65) (end 112.85 78.15) (width 0.4) (layer F.Cu) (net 3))
 (segment (start 130.469998 62.55) (end 114.05 62.55) (width 0.4) (layer F.Cu) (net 3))
 (segment (start 98.45 68.945) (end 97.05 68.945) (width 0.4) (layer F.Cu) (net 3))
 (segment (start 104.845 62.55) (end 98.45 68.945) (width 0.4) (layer F.Cu) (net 3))
 (segment (start 114.05 62.55) (end 104.845 62.55) (width 0.4) (layer F.Cu) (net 3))
 (segment (start 112.15 62.55) (end 112.15 64.65) (width 0.4) (layer F.Cu) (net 3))
 (segment (start 114.05 62.55) (end 112.15 62.55) (width 0.4) (layer F.Cu) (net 3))
 (segment (start 122.5 81.4) (end 122.5 82.6) (width 0.4) (layer F.Cu) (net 3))
 (segment (start 122.5 62.55) (end 122.5 81.4) (width 0.4) (layer F.Cu) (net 3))
 (segment (start 130.469998 62.55) (end 122.5 62.55) (width 0.4) (layer F.Cu) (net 3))
 (segment (start 116.15 79.05) (end 116.15 78.05) (width 0.4) (layer F.Cu) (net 3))
 (segment (start 119.7 82.6) (end 116.15 79.05) (width 0.4) (layer F.Cu) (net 3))
 (segment (start 122.5 82.6) (end 119.7 82.6) (width 0.4) (layer F.Cu) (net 3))
 (segment (start 150 83.7) (end 153.4 87.1) (width 0.4) (layer F.Cu) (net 3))
 (segment (start 131.2 83.7) (end 150 83.7) (width 0.4) (layer F.Cu) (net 3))
 (segment (start 129.4 85.5) (end 131.2 83.7) (width 0.4) (layer F.Cu) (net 3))
 (segment (start 123.95 85.5) (end 129.4 85.5) (width 0.4) (layer F.Cu) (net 3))
 (segment (start 122.5 84.05) (end 123.95 85.5) (width 0.4) (layer F.Cu) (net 3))
 (segment (start 153.4 87.1) (end 154.8 87.1) (width 0.4) (layer F.Cu) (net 3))
 (segment (start 122.5 82.6) (end 122.5 84.05) (width 0.4) (layer F.Cu) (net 3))
 (segment (start 116.15 68.05) (end 114.25 68.05) (width 0.4) (layer F.Cu) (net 5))
 (segment (start 113.91138 64.38862) (end 113.91138 68.05) (width 0.4) (layer F.Cu) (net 5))
 (segment (start 114.25 64.05) (end 113.91138 64.38862) (width 0.4) (layer F.Cu) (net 5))
 (segment (start 116.15 64.05) (end 114.25 64.05) (width 0.4) (layer F.Cu) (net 5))
 (segment (start 113.91138 68.05) (end 112.15 68.05) (width 0.4) (layer F.Cu) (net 5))
 (segment (start 114.25 68.05) (end 113.91138 68.05) (width 0.4) (layer F.Cu) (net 5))
 (segment (start 141.825001 69.524999) (end 141.9 69.45) (width 0.4) (layer F.Cu) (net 13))
 (segment (start 141.825001 71.524999) (end 141.825001 69.524999) (width 0.4) (layer F.Cu) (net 13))
 (segment (start 140.9 72.45) (end 141.825001 71.524999) (width 0.4) (layer F.Cu) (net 13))
 (segment (start 135.75 72.45) (end 140.9 72.45) (width 0.4) (layer F.Cu) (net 13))
 (segment (start 133.35 70.05) (end 135.75 72.45) (width 0.4) (layer F.Cu) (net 13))
 (segment (start 132.15 70.05) (end 133.35 70.05) (width 0.4) (layer F.Cu) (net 13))
 (segment (start 115.75 74.45) (end 116.15 74.05) (width 0.4) (layer F.Cu) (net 9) (status 30))
 (segment (start 112.35 73.85) (end 112.35 75.25) (width 0.4) (layer F.Cu) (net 9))
 (segment (start 112.35 72.275) (end 112.35 73.85) (width 0.4) (layer F.Cu) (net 9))
 (segment (start 107.75 67.675) (end 112.35 72.275) (width 0.4) (layer F.Cu) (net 9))
 (segment (start 106.35 67.675) (end 107.75 67.675) (width 0.4) (layer F.Cu) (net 9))
 (segment (start 113.55 74.05) (end 112.35 75.25) (width 0.4) (layer F.Cu) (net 9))
 (segment (start 116.15 74.05) (end 113.55 74.05) (width 0.4) (layer F.Cu) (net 9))
 (segment (start 116.15 76.05) (end 114.4 76.05) (width 0.4) (layer F.Cu) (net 10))
 (segment (start 114.4 76.05) (end 113.599999 76.850001) (width 0.4) (layer F.Cu) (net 10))
 (segment (start 113.599999 76.850001) (end 110.200001 76.850001) (width 0.4) (layer F.Cu) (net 10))
 (segment (start 110.200001 76.850001) (end 110 76.65) (width 0.4) (layer F.Cu) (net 10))
 (segment (start 110 76.65) (end 110 75.25) (width 0.4) (layer F.Cu) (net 10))
 (segment (start 116.15 76.05) (end 114.930002 76.05) (width 0.4) (layer F.Cu) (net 10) (status 30))
 (segment (start 114.95 76.15) (end 114.9 76.1) (width 0.4) (layer F.Cu) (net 10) (status 30))
 (segment (start 115.05 76.05) (end 114.95 76.15) (width 0.4) (layer F.Cu) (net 10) (status 30))
 (segment (start 116.15 76.05) (end 115.05 76.05) (width 0.4) (layer F.Cu) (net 10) (status 30))
 (segment (start 110 73.85) (end 110 75.25) (width 0.4) (layer F.Cu) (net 10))
 (segment (start 110 71.195) (end 110 73.85) (width 0.4) (layer F.Cu) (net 10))
 (segment (start 107.75 68.945) (end 110 71.195) (width 0.4) (layer F.Cu) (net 10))
 (segment (start 106.35 68.945) (end 107.75 68.945) (width 0.4) (layer F.Cu) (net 10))
 (segment (start 139 76.7) (end 139.2 76.9) (width 0.4) (layer F.Cu) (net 11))
 (segment (start 138.35 76.05) (end 139.2 76.9) (width 0.4) (layer F.Cu) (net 11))
 (segment (start 132.15 76.05) (end 138.35 76.05) (width 0.4) (layer F.Cu) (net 11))
 (segment (start 152.700001 85.000001) (end 159.299999 85.000001) (width 0.4) (layer F.Cu) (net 12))
 (segment (start 150.5 82.8) (end 152.700001 85.000001) (width 0.4) (layer F.Cu) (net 12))
 (segment (start 130.7 82.8) (end 150.5 82.8) (width 0.4) (layer F.Cu) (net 12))
 (segment (start 128.95 84.55) (end 130.7 82.8) (width 0.4) (layer F.Cu) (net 12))
 (segment (start 124.969998 84.55) (end 128.95 84.55) (width 0.4) (layer F.Cu) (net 12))
 (segment (start 124.2 83.780002) (end 124.969998 84.55) (width 0.4) (layer F.Cu) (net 12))
 (segment (start 124.2 78.1) (end 124.2 83.780002) (width 0.4) (layer F.Cu) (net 12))
 (segment (start 159.299999 85.000001) (end 161.4 85) (width 0.4) (layer F.Cu) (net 12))
 (segment (start 130.25 72.05) (end 124.2 78.1) (width 0.4) (layer F.Cu) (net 12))
 (segment (start 132.15 72.05) (end 130.25 72.05) (width 0.4) (layer F.Cu) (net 12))
 (segment (start 134.469998 66.05) (end 136.209998 67.79) (width 0.4) (layer F.Cu) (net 15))
 (segment (start 136.209998 67.79) (end 137 67.79) (width 0.4) (layer F.Cu) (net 15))
 (segment (start 132.15 66.05) (end 134.469998 66.05) (width 0.4) (layer F.Cu) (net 15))
 (segment (start 136.6 64.85) (end 137 65.25) (width 0.4) (layer F.Cu) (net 16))
 (segment (start 134.05 64.05) (end 132.15 64.05) (width 0.4) (layer F.Cu) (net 16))
 (segment (start 134.15 64.05) (end 134.05 64.05) (width 0.4) (layer F.Cu) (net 16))
 (segment (start 135.35 65.25) (end 134.15 64.05) (width 0.4) (layer F.Cu) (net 16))
 (segment (start 137 65.25) (end 135.35 65.25) (width 0.4) (layer F.Cu) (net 16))
 (segment (start 132.15 74.05) (end 140.1 74.05) (width 0.4) (layer F.Cu) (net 17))
 (segment (start 140.1 74.05) (end 141.55 75.5) (width 0.4) (layer F.Cu) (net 17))
 (segment (start 141.55 75.5) (end 141.55 76.9) (width 0.4) (layer F.Cu) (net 17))
 (segment (start 157.7 65.5) (end 162.25 65.5) (width 0.4) (layer F.Cu) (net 18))
 (segment (start 162.25 65.5) (end 162.9 66.15) (width 0.4) (layer F.Cu) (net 18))
 (segment (start 161.1 87.2) (end 161.4 87.5) (width 0.4) (layer F.Cu) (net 19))
 (segment (start 158.2 87.1) (end 158.3 87.2) (width 0.4) (layer F.Cu) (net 19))
 (segment (start 158.6 87.5) (end 158.2 87.1) (width 0.4) (layer F.Cu) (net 19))
 (segment (start 161.4 87.5) (end 158.6 87.5) (width 0.4) (layer F.Cu) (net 19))
 (segment (start 158 83.6) (end 158.2 83.6) (width 0.4) (layer F.Cu) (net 20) (status 30))
 (segment (start 161.4 83.4) (end 161.4 82.5) (width 0.4) (layer F.Cu) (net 20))
 (segment (start 161.2 83.6) (end 161.4 83.4) (width 0.4) (layer F.Cu) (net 20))
 (segment (start 158.2 83.6) (end 161.2 83.6) (width 0.4) (layer F.Cu) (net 20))
 (segment (start 146.75 68.9) (end 151.9 68.9) (width 0.4) (layer F.Cu) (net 21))
 (segment (start 151.9 68.9) (end 152 68.8) (width 0.4) (layer F.Cu) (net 21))
 (segment (start 141.9 66.625) (end 141.9 66.15) (width 0.4) (layer F.Cu) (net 22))
 (segment (start 146.1 66.15) (end 146.75 65.5) (width 0.4) (layer F.Cu) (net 22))
 (segment (start 141.9 66.15) (end 146.1 66.15) (width 0.4) (layer F.Cu) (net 22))
 (segment (start 141.55 80.3) (end 145.25 80.3) (width 0.4) (layer F.Cu) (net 4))
 (segment (start 145.25 80.780002) (end 145.25 80.3) (width 0.4) (layer F.Cu) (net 4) (status 30)))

